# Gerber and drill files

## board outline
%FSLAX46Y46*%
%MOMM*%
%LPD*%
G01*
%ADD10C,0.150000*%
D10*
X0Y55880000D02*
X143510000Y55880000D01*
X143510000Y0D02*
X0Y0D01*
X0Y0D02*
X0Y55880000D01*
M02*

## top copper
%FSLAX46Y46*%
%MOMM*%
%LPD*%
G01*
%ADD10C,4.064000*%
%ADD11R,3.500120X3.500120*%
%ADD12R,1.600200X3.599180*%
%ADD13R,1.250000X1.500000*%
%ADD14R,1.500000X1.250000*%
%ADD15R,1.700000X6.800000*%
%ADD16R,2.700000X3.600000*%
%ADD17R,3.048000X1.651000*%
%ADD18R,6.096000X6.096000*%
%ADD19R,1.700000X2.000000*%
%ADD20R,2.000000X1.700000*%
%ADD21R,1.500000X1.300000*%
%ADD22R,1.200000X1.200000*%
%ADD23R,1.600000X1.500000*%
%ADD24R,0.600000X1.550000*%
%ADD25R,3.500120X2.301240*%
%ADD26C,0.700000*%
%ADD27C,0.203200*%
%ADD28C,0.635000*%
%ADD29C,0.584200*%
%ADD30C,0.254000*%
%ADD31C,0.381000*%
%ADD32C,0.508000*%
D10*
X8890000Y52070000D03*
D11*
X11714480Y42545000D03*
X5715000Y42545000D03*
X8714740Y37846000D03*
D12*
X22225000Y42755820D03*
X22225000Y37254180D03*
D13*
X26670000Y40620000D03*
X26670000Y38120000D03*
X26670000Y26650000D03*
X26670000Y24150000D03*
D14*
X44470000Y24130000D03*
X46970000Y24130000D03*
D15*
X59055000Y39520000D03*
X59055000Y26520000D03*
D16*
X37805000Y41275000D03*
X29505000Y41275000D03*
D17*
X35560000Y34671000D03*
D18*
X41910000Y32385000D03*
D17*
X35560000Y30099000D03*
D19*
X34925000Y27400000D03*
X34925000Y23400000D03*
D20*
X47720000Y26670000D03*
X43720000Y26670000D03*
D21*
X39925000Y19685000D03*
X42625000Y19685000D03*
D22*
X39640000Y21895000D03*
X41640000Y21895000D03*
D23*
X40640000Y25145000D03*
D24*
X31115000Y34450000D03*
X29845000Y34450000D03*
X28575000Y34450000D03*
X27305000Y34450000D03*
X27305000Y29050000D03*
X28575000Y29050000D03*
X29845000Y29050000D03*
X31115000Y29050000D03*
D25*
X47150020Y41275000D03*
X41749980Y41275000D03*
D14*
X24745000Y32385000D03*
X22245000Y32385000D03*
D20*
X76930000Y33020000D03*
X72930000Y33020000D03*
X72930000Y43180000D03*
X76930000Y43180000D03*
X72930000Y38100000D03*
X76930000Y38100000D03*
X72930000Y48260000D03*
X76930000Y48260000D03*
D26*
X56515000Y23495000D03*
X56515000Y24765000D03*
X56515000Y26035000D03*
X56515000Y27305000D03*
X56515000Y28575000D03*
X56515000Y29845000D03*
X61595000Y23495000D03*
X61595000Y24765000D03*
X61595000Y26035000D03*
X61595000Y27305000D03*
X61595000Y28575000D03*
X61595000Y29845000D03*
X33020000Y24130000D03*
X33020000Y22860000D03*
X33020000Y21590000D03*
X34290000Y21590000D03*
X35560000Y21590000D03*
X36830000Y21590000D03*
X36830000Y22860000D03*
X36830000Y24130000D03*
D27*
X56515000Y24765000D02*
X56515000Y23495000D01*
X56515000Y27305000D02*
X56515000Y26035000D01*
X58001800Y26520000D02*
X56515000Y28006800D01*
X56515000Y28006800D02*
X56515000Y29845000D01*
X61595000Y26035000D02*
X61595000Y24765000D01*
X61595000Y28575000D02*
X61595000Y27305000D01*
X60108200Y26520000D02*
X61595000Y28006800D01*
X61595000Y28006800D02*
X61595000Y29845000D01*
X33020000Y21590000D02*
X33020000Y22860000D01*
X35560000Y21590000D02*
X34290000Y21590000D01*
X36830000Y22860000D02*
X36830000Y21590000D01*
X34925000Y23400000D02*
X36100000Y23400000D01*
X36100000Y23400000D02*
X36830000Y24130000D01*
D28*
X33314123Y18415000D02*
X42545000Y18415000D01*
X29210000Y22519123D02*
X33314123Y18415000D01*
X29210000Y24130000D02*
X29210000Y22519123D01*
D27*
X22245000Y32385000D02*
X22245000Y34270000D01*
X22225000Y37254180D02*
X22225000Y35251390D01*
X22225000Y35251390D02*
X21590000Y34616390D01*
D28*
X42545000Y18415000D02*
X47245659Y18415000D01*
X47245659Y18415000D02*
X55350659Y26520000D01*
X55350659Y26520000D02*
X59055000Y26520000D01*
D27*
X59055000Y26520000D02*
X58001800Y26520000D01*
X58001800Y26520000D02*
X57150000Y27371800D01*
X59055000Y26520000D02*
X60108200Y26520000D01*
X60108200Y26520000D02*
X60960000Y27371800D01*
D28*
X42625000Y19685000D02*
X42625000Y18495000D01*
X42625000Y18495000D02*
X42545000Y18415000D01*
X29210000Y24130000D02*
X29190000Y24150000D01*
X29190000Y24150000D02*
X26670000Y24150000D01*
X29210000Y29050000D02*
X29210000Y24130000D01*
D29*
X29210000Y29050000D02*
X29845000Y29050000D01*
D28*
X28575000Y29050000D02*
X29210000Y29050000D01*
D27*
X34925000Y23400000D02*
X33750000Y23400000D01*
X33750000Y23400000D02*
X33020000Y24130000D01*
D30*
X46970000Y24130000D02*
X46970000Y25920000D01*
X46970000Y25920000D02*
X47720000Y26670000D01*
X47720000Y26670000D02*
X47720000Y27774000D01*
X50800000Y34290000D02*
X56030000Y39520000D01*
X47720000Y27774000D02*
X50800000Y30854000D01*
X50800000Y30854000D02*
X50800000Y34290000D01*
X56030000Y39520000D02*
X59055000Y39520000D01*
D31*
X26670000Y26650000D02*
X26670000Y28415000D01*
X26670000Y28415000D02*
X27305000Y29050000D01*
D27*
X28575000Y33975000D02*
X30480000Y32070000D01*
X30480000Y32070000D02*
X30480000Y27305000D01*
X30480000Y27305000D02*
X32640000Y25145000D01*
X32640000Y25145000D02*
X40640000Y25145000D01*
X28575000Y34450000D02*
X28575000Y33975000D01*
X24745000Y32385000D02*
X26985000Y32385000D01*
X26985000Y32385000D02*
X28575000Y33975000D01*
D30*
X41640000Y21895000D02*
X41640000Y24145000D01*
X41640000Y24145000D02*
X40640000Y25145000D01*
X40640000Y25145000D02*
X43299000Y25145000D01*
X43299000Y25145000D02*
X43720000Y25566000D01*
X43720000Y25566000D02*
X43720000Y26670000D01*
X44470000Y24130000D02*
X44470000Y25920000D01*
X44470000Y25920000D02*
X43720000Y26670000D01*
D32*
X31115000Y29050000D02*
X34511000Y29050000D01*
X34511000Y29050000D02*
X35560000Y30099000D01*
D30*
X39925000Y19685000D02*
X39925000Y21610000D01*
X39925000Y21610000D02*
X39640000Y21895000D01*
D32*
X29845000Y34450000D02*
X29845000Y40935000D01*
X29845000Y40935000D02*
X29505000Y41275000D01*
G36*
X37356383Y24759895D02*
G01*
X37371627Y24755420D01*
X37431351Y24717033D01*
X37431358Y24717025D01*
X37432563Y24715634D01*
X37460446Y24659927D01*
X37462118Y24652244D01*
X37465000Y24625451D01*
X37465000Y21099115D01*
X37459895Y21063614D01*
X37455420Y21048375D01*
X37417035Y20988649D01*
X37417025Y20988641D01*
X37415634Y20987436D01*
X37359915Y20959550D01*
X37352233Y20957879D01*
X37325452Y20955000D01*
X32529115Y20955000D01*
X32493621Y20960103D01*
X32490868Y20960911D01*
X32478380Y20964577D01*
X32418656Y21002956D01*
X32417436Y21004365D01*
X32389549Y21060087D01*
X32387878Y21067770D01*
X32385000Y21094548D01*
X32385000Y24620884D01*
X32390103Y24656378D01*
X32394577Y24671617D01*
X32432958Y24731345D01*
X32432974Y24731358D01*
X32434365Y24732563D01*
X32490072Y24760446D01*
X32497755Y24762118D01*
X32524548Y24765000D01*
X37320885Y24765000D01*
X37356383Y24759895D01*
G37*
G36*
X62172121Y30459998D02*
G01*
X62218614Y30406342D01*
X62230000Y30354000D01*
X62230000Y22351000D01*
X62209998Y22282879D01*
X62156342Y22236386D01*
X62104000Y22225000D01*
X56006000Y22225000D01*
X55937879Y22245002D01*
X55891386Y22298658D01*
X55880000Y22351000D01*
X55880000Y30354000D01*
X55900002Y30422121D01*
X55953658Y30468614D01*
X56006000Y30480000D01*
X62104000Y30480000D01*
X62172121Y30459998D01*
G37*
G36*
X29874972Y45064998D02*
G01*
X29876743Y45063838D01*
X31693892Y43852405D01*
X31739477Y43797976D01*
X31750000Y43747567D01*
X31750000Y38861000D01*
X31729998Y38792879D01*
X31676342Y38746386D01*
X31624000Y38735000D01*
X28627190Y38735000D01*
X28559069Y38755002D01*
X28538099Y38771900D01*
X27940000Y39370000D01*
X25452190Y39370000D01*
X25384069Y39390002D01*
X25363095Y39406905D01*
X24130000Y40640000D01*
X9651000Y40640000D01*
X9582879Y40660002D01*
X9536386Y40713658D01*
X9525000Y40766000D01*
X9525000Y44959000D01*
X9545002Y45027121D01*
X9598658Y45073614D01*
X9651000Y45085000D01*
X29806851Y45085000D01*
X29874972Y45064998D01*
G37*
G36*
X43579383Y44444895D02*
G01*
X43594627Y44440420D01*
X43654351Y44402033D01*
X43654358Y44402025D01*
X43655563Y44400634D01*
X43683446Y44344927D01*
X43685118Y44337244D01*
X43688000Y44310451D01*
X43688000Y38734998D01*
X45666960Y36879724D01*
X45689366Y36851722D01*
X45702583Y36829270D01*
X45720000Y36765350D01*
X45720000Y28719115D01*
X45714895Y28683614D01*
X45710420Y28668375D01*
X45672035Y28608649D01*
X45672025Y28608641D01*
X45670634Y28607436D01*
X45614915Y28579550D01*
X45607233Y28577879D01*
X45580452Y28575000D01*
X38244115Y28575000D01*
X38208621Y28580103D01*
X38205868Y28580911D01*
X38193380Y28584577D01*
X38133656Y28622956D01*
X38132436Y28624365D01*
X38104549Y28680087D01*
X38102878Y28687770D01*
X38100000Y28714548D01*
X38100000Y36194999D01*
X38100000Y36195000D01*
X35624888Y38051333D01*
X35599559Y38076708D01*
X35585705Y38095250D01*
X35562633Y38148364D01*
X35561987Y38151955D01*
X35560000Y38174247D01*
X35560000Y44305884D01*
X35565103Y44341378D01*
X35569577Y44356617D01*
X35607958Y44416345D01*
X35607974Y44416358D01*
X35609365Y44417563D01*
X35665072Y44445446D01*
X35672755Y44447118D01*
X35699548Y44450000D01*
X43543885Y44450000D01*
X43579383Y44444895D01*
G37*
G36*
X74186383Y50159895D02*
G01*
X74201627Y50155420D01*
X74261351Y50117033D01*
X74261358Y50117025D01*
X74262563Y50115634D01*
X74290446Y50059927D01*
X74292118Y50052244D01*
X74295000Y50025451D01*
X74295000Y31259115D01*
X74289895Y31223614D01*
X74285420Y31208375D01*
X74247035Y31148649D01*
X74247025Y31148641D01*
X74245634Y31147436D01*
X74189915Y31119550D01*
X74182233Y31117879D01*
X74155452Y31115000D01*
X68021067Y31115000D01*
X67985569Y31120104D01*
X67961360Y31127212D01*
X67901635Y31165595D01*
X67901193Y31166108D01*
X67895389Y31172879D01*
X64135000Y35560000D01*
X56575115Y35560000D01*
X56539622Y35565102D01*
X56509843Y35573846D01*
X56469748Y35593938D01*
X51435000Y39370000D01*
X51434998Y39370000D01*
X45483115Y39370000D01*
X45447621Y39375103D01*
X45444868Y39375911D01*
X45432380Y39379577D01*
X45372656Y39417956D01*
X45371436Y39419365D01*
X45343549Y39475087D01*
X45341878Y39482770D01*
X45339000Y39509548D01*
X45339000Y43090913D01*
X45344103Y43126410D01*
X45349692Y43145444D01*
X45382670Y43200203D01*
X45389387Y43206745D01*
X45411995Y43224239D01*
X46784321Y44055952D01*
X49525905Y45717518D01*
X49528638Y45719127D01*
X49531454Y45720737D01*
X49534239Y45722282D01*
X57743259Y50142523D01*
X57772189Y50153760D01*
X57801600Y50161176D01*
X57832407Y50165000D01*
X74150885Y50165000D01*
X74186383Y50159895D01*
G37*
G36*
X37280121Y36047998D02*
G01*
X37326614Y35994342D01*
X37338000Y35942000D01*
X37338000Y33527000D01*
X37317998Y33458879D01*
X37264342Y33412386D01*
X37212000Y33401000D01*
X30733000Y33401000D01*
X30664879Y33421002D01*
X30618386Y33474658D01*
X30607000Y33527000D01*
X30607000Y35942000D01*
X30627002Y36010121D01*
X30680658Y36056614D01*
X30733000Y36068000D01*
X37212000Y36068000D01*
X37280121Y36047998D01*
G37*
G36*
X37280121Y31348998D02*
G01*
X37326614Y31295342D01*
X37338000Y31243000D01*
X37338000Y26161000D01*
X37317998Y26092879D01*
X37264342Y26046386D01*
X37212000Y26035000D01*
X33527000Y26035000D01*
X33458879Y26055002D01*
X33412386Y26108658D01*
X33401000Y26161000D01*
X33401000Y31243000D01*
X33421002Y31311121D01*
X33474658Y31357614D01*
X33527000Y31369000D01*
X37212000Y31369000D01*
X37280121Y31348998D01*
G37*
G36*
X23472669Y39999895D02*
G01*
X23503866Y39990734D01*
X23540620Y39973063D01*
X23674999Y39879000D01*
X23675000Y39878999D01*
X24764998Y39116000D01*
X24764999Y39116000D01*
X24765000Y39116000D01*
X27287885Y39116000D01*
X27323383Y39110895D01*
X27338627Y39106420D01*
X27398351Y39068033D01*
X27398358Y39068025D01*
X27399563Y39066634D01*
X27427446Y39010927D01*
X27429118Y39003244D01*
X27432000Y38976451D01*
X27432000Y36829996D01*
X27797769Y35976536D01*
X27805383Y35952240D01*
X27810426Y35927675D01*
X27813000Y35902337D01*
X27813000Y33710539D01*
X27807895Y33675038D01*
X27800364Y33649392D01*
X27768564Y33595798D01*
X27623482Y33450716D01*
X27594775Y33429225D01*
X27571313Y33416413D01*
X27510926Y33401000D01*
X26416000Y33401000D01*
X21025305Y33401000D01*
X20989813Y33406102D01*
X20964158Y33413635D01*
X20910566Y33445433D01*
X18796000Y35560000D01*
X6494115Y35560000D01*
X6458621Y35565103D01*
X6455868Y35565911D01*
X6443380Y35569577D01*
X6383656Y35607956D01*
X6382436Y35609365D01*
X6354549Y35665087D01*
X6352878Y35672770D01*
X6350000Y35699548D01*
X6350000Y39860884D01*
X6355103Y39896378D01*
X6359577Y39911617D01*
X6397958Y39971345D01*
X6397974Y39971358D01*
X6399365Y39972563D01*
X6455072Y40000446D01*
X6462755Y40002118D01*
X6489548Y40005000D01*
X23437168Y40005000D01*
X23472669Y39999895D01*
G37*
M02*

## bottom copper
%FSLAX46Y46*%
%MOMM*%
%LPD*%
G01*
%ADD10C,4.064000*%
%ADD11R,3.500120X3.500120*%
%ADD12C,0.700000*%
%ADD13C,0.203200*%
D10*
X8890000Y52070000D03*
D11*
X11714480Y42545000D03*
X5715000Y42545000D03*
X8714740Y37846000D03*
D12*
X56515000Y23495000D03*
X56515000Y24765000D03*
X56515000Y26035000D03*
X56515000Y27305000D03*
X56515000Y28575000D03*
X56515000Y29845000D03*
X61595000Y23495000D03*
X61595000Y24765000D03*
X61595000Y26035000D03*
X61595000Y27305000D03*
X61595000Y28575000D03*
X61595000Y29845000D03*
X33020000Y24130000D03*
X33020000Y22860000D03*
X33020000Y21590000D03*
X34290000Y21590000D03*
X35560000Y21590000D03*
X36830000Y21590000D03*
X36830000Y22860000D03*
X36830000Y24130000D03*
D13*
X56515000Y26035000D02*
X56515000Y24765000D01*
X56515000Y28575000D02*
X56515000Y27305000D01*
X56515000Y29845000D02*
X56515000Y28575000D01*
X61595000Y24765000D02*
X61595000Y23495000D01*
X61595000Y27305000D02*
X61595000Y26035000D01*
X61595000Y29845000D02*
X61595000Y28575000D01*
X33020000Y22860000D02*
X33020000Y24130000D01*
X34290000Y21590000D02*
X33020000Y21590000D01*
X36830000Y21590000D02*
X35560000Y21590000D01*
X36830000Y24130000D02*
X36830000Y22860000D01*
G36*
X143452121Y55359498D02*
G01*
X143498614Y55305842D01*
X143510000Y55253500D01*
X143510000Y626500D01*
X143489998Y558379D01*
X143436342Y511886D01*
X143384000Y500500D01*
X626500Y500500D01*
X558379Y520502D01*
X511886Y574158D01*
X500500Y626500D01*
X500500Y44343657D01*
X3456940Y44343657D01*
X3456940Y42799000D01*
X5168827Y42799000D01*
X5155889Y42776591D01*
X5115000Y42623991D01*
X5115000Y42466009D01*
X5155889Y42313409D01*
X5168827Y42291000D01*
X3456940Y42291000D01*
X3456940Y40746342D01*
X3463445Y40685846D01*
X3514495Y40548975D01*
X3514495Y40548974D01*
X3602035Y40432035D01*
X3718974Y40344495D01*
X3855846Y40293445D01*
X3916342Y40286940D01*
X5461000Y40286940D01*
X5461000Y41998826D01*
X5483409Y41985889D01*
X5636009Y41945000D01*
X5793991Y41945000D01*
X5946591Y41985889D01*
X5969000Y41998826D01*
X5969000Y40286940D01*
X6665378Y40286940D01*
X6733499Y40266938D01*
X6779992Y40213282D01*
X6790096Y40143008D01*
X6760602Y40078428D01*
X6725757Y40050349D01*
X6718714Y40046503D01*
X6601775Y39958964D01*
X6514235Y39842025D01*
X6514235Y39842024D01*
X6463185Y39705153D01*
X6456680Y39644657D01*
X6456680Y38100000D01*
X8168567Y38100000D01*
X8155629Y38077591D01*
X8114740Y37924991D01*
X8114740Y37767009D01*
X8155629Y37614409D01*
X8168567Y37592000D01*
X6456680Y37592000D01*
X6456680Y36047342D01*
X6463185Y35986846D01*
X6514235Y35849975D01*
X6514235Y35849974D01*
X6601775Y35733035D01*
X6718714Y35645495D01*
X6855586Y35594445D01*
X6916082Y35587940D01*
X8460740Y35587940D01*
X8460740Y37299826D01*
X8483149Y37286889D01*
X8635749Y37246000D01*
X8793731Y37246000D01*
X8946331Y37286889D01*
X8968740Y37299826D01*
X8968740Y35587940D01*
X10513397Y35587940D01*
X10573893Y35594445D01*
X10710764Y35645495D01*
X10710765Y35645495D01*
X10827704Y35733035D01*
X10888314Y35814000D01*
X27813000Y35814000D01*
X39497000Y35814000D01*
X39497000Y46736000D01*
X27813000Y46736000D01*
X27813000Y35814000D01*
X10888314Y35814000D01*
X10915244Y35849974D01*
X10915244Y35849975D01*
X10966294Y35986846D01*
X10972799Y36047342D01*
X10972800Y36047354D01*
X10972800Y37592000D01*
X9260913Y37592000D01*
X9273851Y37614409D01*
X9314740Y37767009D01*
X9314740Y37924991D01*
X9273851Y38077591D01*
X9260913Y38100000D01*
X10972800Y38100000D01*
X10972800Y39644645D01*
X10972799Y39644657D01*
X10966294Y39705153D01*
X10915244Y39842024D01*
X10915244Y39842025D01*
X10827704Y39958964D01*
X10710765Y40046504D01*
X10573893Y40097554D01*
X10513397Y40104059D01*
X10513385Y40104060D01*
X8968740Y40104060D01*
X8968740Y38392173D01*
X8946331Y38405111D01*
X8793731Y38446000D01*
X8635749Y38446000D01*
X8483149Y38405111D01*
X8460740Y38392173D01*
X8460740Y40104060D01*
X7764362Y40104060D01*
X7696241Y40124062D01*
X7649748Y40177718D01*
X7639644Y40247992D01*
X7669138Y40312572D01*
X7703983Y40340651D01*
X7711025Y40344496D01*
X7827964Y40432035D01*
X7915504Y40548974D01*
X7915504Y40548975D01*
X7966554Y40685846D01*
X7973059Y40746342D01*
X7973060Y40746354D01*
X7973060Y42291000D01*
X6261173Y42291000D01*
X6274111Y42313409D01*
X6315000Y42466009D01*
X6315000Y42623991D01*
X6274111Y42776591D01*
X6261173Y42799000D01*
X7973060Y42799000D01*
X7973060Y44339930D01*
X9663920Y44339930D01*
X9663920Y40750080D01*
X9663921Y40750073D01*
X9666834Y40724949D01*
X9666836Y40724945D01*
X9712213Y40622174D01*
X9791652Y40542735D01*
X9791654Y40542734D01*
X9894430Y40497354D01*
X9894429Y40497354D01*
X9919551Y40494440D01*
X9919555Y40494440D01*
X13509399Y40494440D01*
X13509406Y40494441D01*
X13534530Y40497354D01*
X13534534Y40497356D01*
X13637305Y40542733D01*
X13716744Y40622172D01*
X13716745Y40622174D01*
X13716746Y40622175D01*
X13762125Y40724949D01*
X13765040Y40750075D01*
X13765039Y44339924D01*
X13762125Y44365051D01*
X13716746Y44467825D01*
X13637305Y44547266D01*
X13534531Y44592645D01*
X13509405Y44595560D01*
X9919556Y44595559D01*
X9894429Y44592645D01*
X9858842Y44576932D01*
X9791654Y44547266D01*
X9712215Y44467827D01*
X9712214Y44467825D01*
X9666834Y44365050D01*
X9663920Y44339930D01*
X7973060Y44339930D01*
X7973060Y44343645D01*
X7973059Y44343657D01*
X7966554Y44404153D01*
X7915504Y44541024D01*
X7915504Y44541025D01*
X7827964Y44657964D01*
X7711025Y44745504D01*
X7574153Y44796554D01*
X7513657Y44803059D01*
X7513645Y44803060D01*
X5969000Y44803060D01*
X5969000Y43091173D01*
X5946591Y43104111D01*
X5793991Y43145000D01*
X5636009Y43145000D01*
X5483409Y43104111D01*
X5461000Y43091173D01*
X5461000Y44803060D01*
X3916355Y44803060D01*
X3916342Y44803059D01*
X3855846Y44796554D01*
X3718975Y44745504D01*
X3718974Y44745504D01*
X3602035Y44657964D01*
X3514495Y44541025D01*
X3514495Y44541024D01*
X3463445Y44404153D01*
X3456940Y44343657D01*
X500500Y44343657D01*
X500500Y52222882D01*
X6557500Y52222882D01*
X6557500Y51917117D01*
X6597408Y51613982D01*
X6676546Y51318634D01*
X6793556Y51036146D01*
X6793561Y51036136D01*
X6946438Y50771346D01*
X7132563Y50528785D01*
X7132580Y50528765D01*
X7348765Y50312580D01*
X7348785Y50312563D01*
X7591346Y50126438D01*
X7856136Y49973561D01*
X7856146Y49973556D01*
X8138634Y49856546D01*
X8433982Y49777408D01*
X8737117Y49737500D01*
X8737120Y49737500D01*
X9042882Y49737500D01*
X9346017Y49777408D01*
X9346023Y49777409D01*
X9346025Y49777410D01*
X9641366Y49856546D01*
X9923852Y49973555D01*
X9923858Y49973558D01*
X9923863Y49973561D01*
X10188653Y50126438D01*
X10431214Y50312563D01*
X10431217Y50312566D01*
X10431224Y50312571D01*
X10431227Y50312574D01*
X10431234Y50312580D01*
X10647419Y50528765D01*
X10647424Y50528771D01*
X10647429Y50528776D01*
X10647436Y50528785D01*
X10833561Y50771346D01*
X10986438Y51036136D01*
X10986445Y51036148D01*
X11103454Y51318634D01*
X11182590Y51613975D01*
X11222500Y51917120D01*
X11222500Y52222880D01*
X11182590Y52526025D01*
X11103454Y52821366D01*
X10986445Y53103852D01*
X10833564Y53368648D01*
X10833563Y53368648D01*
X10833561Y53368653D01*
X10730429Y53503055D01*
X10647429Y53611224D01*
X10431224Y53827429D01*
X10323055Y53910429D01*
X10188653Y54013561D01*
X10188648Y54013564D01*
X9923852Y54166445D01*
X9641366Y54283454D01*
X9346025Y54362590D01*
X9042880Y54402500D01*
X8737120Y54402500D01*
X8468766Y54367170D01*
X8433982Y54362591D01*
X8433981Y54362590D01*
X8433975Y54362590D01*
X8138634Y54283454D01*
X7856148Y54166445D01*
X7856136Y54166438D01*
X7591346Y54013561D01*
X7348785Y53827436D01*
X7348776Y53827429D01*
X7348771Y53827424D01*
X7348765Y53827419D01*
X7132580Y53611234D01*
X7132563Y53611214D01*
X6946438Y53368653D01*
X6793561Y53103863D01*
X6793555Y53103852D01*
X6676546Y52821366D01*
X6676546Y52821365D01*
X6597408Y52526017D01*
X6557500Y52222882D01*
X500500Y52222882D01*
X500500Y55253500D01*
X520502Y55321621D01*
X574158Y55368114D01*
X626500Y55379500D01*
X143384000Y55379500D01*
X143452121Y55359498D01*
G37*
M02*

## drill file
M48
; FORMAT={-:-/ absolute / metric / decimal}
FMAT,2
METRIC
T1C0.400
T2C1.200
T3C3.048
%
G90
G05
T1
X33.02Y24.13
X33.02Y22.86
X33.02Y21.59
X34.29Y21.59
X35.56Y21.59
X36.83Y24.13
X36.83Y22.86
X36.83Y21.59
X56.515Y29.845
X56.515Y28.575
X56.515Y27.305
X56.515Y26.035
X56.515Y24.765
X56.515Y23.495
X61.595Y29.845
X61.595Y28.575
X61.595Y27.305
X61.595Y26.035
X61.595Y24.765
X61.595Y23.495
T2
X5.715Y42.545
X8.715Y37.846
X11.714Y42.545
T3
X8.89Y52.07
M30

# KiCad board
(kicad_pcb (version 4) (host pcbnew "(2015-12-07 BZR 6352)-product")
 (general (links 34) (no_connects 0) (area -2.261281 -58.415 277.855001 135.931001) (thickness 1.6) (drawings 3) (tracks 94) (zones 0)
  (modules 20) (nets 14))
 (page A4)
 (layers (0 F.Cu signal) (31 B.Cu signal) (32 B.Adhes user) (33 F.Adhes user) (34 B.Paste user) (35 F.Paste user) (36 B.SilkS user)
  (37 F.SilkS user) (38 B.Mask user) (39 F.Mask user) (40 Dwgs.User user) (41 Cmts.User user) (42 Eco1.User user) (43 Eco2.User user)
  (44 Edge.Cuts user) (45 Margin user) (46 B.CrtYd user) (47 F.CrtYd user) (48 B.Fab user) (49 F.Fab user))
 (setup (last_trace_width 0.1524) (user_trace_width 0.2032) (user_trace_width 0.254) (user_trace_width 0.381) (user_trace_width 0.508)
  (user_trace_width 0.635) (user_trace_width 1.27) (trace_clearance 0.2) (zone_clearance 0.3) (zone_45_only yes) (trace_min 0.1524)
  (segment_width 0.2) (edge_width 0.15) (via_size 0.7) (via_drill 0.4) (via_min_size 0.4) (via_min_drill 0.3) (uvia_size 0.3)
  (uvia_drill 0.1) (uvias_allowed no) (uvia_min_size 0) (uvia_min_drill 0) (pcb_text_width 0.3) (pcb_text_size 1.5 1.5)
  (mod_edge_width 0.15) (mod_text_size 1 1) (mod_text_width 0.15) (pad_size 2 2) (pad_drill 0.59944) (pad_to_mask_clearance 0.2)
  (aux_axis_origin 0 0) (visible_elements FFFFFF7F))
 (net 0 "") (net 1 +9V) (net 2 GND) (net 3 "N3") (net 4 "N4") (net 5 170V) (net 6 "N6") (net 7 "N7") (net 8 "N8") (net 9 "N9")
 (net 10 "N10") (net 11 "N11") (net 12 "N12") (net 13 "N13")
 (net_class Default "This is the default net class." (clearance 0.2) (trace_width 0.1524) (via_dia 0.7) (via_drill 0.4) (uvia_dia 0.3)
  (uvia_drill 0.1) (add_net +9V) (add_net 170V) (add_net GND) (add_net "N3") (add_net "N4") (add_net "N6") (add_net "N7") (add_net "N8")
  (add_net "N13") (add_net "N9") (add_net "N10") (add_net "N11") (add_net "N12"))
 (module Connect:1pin (layer F.Cu) (at 8.89 -52.07)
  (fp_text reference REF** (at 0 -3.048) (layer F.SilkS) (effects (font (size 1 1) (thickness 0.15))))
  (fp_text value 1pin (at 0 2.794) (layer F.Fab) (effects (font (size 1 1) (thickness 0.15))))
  (pad 1 thru_hole circle (at 0 0) (size 4.064 4.064) (drill 3.048) (layers *.Cu *.Mask F.SilkS)))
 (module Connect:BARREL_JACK (layer F.Cu) (at 5.51434 -42.545)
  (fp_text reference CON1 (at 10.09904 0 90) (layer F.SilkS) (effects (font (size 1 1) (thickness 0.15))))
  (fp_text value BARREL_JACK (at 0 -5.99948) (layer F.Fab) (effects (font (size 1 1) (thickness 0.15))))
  (pad 1 thru_hole rect (at 6.20014 0) (size 3.50012 3.50012) (drill 1.2) (layers *.Cu *.Mask F.SilkS) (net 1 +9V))
  (pad 2 thru_hole rect (at 0.20066 0) (size 3.50012 3.50012) (drill 1.2) (layers *.Cu *.Mask F.SilkS) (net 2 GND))
  (pad 3 thru_hole rect (at 3.2004 4.699) (size 3.50012 3.50012) (drill 1.2) (layers *.Cu *.Mask F.SilkS) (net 2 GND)))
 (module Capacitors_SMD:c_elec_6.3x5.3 (layer F.Cu) (at 22.225 -40.005 90)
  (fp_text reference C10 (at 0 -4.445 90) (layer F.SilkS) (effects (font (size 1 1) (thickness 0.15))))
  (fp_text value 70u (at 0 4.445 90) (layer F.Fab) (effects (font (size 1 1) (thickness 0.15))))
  (pad 1 smd rect (at 2.75082 0 90) (size 3.59918 1.6002) (layers F.Cu F.Paste F.Mask) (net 1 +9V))
  (pad 2 smd rect (at -2.75082 0 90) (size 3.59918 1.6002) (layers F.Cu F.Paste F.Mask) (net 2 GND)))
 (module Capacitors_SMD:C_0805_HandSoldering (layer F.Cu) (at 26.67 -39.37 270)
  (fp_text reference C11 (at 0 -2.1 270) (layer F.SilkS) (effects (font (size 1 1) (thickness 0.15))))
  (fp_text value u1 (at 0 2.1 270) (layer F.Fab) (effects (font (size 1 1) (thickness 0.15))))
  (pad 1 smd rect (at -1.25 0 270) (size 1.5 1.25) (layers F.Cu F.Paste F.Mask) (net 1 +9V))
  (pad 2 smd rect (at 1.25 0 270) (size 1.5 1.25) (layers F.Cu F.Paste F.Mask) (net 2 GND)))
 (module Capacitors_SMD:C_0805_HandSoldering (layer F.Cu) (at 26.67 -25.4 270)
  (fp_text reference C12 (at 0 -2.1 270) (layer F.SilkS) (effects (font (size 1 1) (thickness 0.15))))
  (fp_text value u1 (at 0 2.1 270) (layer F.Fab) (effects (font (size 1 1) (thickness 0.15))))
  (pad 1 smd rect (at -1.25 0 270) (size 1.5 1.25) (layers F.Cu F.Paste F.Mask) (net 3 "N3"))
  (pad 2 smd rect (at 1.25 0 270) (size 1.5 1.25) (layers F.Cu F.Paste F.Mask) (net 2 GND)))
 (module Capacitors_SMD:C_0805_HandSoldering (layer F.Cu) (at 45.72 -24.13)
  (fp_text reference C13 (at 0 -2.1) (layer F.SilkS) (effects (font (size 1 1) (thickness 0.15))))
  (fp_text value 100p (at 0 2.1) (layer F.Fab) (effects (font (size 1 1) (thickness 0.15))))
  (pad 1 smd rect (at -1.25 0) (size 1.5 1.25) (layers F.Cu F.Paste F.Mask) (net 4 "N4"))
  (pad 2 smd rect (at 1.25 0) (size 1.5 1.25) (layers F.Cu F.Paste F.Mask) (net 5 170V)))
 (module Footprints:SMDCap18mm (layer F.Cu) (at 59.055 -33.02 180)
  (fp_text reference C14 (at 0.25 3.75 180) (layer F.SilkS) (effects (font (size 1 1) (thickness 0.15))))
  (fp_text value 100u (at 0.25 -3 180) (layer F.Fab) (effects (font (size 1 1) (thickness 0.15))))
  (pad 1 smd rect (at 0 6.5 180) (size 1.7 6.8) (layers F.Cu F.Paste F.Mask) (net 5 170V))
  (pad 2 smd rect (at 0 -6.5 180) (size 1.7 6.8) (layers F.Cu F.Paste F.Mask) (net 2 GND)))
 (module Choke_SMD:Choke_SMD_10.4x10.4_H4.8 (layer F.Cu) (at 33.655 -41.275 180)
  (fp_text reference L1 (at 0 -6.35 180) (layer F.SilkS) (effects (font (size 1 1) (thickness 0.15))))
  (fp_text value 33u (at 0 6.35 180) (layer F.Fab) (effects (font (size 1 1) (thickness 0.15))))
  (pad 1 smd rect (at -4.15 0 180) (size 2.7 3.6) (layers F.Cu F.Paste F.Mask) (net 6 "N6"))
  (pad 2 smd rect (at 4.15 0 180) (size 2.7 3.6) (layers F.Cu F.Paste F.Mask) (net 1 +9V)))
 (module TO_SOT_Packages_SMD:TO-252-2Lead (layer F.Cu) (at 35.56 -32.385 270)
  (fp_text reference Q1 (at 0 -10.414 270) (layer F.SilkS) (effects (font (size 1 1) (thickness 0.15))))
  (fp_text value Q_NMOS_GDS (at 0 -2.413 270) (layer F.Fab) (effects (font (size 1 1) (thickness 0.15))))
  (pad 1 smd rect (at -2.286 0 270) (size 1.651 3.048) (layers F.Cu F.Paste F.Mask) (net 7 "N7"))
  (pad 2 smd rect (at 0 -6.35 270) (size 6.096 6.096) (layers F.Cu F.Paste F.Mask) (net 6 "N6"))
  (pad 3 smd rect (at 2.286 0 270) (size 1.651 3.048) (layers F.Cu F.Paste F.Mask) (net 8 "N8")))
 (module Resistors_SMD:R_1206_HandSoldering (layer F.Cu) (at 34.925 -25.4 270)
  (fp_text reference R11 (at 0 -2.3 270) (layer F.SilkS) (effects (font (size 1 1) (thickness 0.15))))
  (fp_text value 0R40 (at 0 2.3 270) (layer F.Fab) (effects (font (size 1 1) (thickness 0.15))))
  (pad 1 smd rect (at -2 0 270) (size 2 1.7) (layers F.Cu F.Paste F.Mask) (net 8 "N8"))
  (pad 2 smd rect (at 2 0 270) (size 2 1.7) (layers F.Cu F.Paste F.Mask) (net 2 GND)))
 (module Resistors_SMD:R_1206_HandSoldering (layer F.Cu) (at 45.72 -26.67 180)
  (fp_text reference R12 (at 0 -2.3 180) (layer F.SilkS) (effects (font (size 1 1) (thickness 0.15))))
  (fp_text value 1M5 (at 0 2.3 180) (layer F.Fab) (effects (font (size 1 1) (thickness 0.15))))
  (pad 1 smd rect (at -2 0 180) (size 2 1.7) (layers F.Cu F.Paste F.Mask) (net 5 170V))
  (pad 2 smd rect (at 2 0 180) (size 2 1.7) (layers F.Cu F.Paste F.Mask) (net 4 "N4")))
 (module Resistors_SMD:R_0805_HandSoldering (layer F.Cu) (at 41.275 -19.685)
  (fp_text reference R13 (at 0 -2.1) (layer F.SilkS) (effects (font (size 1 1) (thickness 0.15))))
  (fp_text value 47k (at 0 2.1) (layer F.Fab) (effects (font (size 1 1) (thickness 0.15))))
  (pad 1 smd rect (at -1.35 0) (size 1.5 1.3) (layers F.Cu F.Paste F.Mask) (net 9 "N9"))
  (pad 2 smd rect (at 1.35 0) (size 1.5 1.3) (layers F.Cu F.Paste F.Mask) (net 2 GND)))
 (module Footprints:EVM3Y (layer F.Cu) (at 40.64 -23.495)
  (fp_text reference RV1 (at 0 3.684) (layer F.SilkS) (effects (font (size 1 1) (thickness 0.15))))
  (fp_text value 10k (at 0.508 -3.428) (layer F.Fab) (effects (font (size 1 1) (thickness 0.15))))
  (pad 1 smd rect (at -1 1.6) (size 1.2 1.2) (layers F.Cu F.Paste F.Mask) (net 9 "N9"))
  (pad 3 smd rect (at 1 1.6) (size 1.2 1.2) (layers F.Cu F.Paste F.Mask) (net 4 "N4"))
  (pad 2 smd rect (at 0 -1.65) (size 1.6 1.5) (layers F.Cu F.Paste F.Mask) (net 4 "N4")))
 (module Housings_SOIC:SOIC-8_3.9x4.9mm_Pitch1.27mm (layer F.Cu) (at 29.21 -31.75 270)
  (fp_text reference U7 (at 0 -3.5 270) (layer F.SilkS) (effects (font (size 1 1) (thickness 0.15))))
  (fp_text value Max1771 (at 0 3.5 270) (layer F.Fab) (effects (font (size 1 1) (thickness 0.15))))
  (pad 1 smd rect (at -2.7 -1.905 270) (size 1.55 0.6) (layers F.Cu F.Paste F.Mask) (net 7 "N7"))
  (pad 2 smd rect (at -2.7 -0.635 270) (size 1.55 0.6) (layers F.Cu F.Paste F.Mask) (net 1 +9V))
  (pad 3 smd rect (at -2.7 0.635 270) (size 1.55 0.6) (layers F.Cu F.Paste F.Mask) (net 4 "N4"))
  (pad 4 smd rect (at -2.7 1.905 270) (size 1.55 0.6) (layers F.Cu F.Paste F.Mask) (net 2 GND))
  (pad 5 smd rect (at 2.7 1.905 270) (size 1.55 0.6) (layers F.Cu F.Paste F.Mask) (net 3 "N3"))
  (pad 6 smd rect (at 2.7 0.635 270) (size 1.55 0.6) (layers F.Cu F.Paste F.Mask) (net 2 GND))
  (pad 7 smd rect (at 2.7 -0.635 270) (size 1.55 0.6) (layers F.Cu F.Paste F.Mask) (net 2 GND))
  (pad 8 smd rect (at 2.7 -1.905 270) (size 1.55 0.6) (layers F.Cu F.Paste F.Mask) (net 8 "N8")))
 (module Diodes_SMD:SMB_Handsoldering (layer F.Cu) (at 44.45 -41.275 180)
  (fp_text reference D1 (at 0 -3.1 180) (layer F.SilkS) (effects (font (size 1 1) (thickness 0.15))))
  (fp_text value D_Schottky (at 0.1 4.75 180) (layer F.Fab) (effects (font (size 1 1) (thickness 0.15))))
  (pad 1 smd rect (at -2.70002 0 180) (size 3.50012 2.30124) (layers F.Cu F.Paste F.Mask) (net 5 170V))
  (pad 2 smd rect (at 2.70002 0 180) (size 3.50012 2.30124) (layers F.Cu F.Paste F.Mask) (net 6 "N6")))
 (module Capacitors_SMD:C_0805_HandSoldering (layer F.Cu) (at 23.495 -32.385 180)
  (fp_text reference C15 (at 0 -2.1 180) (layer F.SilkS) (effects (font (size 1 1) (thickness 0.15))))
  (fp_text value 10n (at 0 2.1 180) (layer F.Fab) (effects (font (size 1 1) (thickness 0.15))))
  (pad 1 smd rect (at -1.25 0 180) (size 1.5 1.25) (layers F.Cu F.Paste F.Mask) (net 4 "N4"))
  (pad 2 smd rect (at 1.25 0 180) (size 1.5 1.25) (layers F.Cu F.Paste F.Mask) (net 2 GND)))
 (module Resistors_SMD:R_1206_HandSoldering (layer F.Cu) (at 74.93 -33.02 180)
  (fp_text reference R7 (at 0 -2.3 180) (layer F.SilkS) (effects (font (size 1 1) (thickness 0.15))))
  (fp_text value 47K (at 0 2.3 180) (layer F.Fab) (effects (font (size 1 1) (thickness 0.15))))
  (pad 1 smd rect (at -2 0 180) (size 2 1.7) (layers F.Cu F.Paste F.Mask) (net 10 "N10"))
  (pad 2 smd rect (at 2 0 180) (size 2 1.7) (layers F.Cu F.Paste F.Mask) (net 5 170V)))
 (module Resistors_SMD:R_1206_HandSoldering (layer F.Cu) (at 74.93 -43.18)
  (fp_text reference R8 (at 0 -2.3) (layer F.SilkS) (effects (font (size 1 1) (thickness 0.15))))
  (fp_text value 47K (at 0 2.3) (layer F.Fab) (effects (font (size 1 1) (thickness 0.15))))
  (pad 1 smd rect (at -2 0) (size 2 1.7) (layers F.Cu F.Paste F.Mask) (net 5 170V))
  (pad 2 smd rect (at 2 0) (size 2 1.7) (layers F.Cu F.Paste F.Mask) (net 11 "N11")))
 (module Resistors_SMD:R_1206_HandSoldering (layer F.Cu) (at 74.93 -38.1)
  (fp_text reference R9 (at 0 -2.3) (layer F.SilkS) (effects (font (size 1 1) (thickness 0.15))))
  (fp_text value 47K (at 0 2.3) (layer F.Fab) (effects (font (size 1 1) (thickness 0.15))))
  (pad 1 smd rect (at -2 0) (size 2 1.7) (layers F.Cu F.Paste F.Mask) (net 5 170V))
  (pad 2 smd rect (at 2 0) (size 2 1.7) (layers F.Cu F.Paste F.Mask) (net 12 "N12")))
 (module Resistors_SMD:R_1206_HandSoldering (layer F.Cu) (at 74.93 -48.26)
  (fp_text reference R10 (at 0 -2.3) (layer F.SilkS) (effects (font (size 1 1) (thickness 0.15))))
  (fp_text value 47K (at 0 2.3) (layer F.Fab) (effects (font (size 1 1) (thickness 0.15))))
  (pad 1 smd rect (at -2 0) (size 2 1.7) (layers F.Cu F.Paste F.Mask) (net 5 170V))
  (pad 2 smd rect (at 2 0) (size 2 1.7) (layers F.Cu F.Paste F.Mask) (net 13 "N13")))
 (gr_line (start 0 -55.88) (end 143.51 -55.88) (layer Edge.Cuts) (width 0.15))
 (gr_line (start 143.51 0) (end 0 0) (layer Edge.Cuts) (width 0.15))
 (gr_line (start 0 0) (end 0 -55.88) (layer Edge.Cuts) (width 0.15))
 (segment (start 56.515 -24.765) (end 56.515 -23.495) (width 0.2032) (layer F.Cu) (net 2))
 (via (at 56.515 -23.495) (size 0.7) (drill 0.4) (layers F.Cu B.Cu) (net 2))
 (segment (start 56.515 -26.035) (end 56.515 -24.765) (width 0.2032) (layer B.Cu) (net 2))
 (via (at 56.515 -24.765) (size 0.7) (drill 0.4) (layers F.Cu B.Cu) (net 2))
 (segment (start 56.515 -27.305) (end 56.515 -26.035) (width 0.2032) (layer F.Cu) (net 2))
 (via (at 56.515 -26.035) (size 0.7) (drill 0.4) (layers F.Cu B.Cu) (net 2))
 (segment (start 56.515 -28.575) (end 56.515 -27.305) (width 0.2032) (layer B.Cu) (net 2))
 (via (at 56.515 -27.305) (size 0.7) (drill 0.4) (layers F.Cu B.Cu) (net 2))
 (segment (start 56.515 -29.845) (end 56.515 -28.575) (width 0.2032) (layer B.Cu) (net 2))
 (via (at 56.515 -28.575) (size 0.7) (drill 0.4) (layers F.Cu B.Cu) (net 2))
 (segment (start 58.0018 -26.52) (end 56.515 -28.0068) (width 0.2032) (layer F.Cu) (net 2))
 (segment (start 56.515 -28.0068) (end 56.515 -29.845) (width 0.2032) (layer F.Cu) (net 2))
 (via (at 56.515 -29.845) (size 0.7) (drill 0.4) (layers F.Cu B.Cu) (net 2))
 (segment (start 61.595 -24.765) (end 61.595 -23.495) (width 0.2032) (layer B.Cu) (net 2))
 (via (at 61.595 -23.495) (size 0.7) (drill 0.4) (layers F.Cu B.Cu) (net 2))
 (segment (start 61.595 -26.035) (end 61.595 -24.765) (width 0.2032) (layer F.Cu) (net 2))
 (via (at 61.595 -24.765) (size 0.7) (drill 0.4) (layers F.Cu B.Cu) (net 2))
 (segment (start 61.595 -27.305) (end 61.595 -26.035) (width 0.2032) (layer B.Cu) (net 2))
 (via (at 61.595 -26.035) (size 0.7) (drill 0.4) (layers F.Cu B.Cu) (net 2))
 (segment (start 61.595 -28.575) (end 61.595 -27.305) (width 0.2032) (layer F.Cu) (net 2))
 (via (at 61.595 -27.305) (size 0.7) (drill 0.4) (layers F.Cu B.Cu) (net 2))
 (segment (start 61.595 -29.845) (end 61.595 -28.575) (width 0.2032) (layer B.Cu) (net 2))
 (via (at 61.595 -28.575) (size 0.7) (drill 0.4) (layers F.Cu B.Cu) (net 2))
 (segment (start 60.1082 -26.52) (end 61.595 -28.0068) (width 0.2032) (layer F.Cu) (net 2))
 (segment (start 61.595 -28.0068) (end 61.595 -29.845) (width 0.2032) (layer F.Cu) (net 2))
 (via (at 61.595 -29.845) (size 0.7) (drill 0.4) (layers F.Cu B.Cu) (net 2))
 (segment (start 33.02 -22.86) (end 33.02 -24.13) (width 0.2032) (layer B.Cu) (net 2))
 (via (at 33.02 -24.13) (size 0.7) (drill 0.4) (layers F.Cu B.Cu) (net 2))
 (segment (start 33.02 -21.59) (end 33.02 -22.86) (width 0.2032) (layer F.Cu) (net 2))
 (via (at 33.02 -22.86) (size 0.7) (drill 0.4) (layers F.Cu B.Cu) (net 2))
 (segment (start 34.29 -21.59) (end 33.02 -21.59) (width 0.2032) (layer B.Cu) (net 2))
 (via (at 33.02 -21.59) (size 0.7) (drill 0.4) (layers F.Cu B.Cu) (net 2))
 (segment (start 35.56 -21.59) (end 34.29 -21.59) (width 0.2032) (layer F.Cu) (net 2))
 (via (at 34.29 -21.59) (size 0.7) (drill 0.4) (layers F.Cu B.Cu) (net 2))
 (segment (start 36.83 -21.59) (end 35.56 -21.59) (width 0.2032) (layer B.Cu) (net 2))
 (via (at 35.56 -21.59) (size 0.7) (drill 0.4) (layers F.Cu B.Cu) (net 2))
 (segment (start 36.83 -22.86) (end 36.83 -21.59) (width 0.2032) (layer F.Cu) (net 2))
 (via (at 36.83 -21.59) (size 0.7) (drill 0.4) (layers F.Cu B.Cu) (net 2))
 (segment (start 36.83 -24.13) (end 36.83 -22.86) (width 0.2032) (layer B.Cu) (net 2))
 (via (at 36.83 -22.86) (size 0.7) (drill 0.4) (layers F.Cu B.Cu) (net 2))
 (segment (start 34.925 -23.4) (end 36.1 -23.4) (width 0.2032) (layer F.Cu) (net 2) (status 10))
 (segment (start 36.1 -23.4) (end 36.83 -24.13) (width 0.2032) (layer F.Cu) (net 2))
 (via (at 36.83 -24.13) (size 0.7) (drill 0.4) (layers F.Cu B.Cu) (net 2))
 (segment (start 33.314123 -18.415) (end 42.545 -18.415) (width 0.635) (layer F.Cu) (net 2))
 (segment (start 29.21 -22.519123) (end 33.314123 -18.415) (width 0.635) (layer F.Cu) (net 2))
 (segment (start 29.21 -24.13) (end 29.21 -22.519123) (width 0.635) (layer F.Cu) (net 2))
 (segment (start 22.245 -32.385) (end 22.245 -34.27) (width 0.2032) (layer F.Cu) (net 2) (status 10))
 (segment (start 22.225 -37.25418) (end 22.225 -35.25139) (width 0.2032) (layer F.Cu) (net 2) (status 10))
 (segment (start 22.225 -35.25139) (end 21.59 -34.61639) (width 0.2032) (layer F.Cu) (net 2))
 (segment (start 42.545 -18.415) (end 47.245659 -18.415) (width 0.635) (layer F.Cu) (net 2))
 (segment (start 47.245659 -18.415) (end 55.350659 -26.52) (width 0.635) (layer F.Cu) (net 2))
 (segment (start 55.350659 -26.52) (end 59.055 -26.52) (width 0.635) (layer F.Cu) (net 2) (status 20))
 (segment (start 59.055 -26.52) (end 58.0018 -26.52) (width 0.2032) (layer F.Cu) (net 2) (status 10))
 (segment (start 58.0018 -26.52) (end 57.15 -27.3718) (width 0.2032) (layer F.Cu) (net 2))
 (segment (start 59.055 -26.52) (end 60.1082 -26.52) (width 0.2032) (layer F.Cu) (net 2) (status 10))
 (segment (start 60.1082 -26.52) (end 60.96 -27.3718) (width 0.2032) (layer F.Cu) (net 2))
 (segment (start 42.625 -19.685) (end 42.625 -18.495) (width 0.635) (layer F.Cu) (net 2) (status 10))
 (segment (start 42.625 -18.495) (end 42.545 -18.415) (width 0.635) (layer F.Cu) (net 2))
 (segment (start 29.21 -24.13) (end 29.19 -24.15) (width 0.635) (layer F.Cu) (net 2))
 (segment (start 29.19 -24.15) (end 26.67 -24.15) (width 0.635) (layer F.Cu) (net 2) (status 20))
 (segment (start 29.21 -29.05) (end 29.21 -24.13) (width 0.635) (layer F.Cu) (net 2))
 (segment (start 29.21 -29.05) (end 29.845 -29.05) (width 0.5842) (layer F.Cu) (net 2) (status 20))
 (segment (start 28.575 -29.05) (end 29.21 -29.05) (width 0.635) (layer F.Cu) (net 2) (status 10))
 (segment (start 34.925 -23.4) (end 33.75 -23.4) (width 0.2032) (layer F.Cu) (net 2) (status 10))
 (segment (start 33.75 -23.4) (end 33.02 -24.13) (width 0.2032) (layer F.Cu) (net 2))
 (segment (start 46.97 -24.13) (end 46.97 -25.92) (width 0.254) (layer F.Cu) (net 5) (status 30))
 (segment (start 46.97 -25.92) (end 47.72 -26.67) (width 0.254) (layer F.Cu) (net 5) (status 30))
 (segment (start 47.72 -26.67) (end 47.72 -27.774) (width 0.254) (layer F.Cu) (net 5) (status 10))
 (segment (start 50.8 -34.29) (end 56.03 -39.52) (width 0.254) (layer F.Cu) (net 5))
 (segment (start 47.72 -27.774) (end 50.8 -30.854) (width 0.254) (layer F.Cu) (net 5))
 (segment (start 50.8 -30.854) (end 50.8 -34.29) (width 0.254) (layer F.Cu) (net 5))
 (segment (start 56.03 -39.52) (end 59.055 -39.52) (width 0.254) (layer F.Cu) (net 5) (status 20))
 (segment (start 26.67 -26.65) (end 26.67 -28.415) (width 0.381) (layer F.Cu) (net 3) (status 10))
 (segment (start 26.67 -28.415) (end 27.305 -29.05) (width 0.381) (layer F.Cu) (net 3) (status 20))
 (segment (start 28.575 -33.975) (end 30.48 -32.07) (width 0.2032) (layer F.Cu) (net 4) (status 10))
 (segment (start 30.48 -32.07) (end 30.48 -27.305) (width 0.2032) (layer F.Cu) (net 4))
 (segment (start 30.48 -27.305) (end 32.64 -25.145) (width 0.2032) (layer F.Cu) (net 4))
 (segment (start 32.64 -25.145) (end 40.64 -25.145) (width 0.2032) (layer F.Cu) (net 4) (status 20))
 (segment (start 28.575 -34.45) (end 28.575 -33.975) (width 0.2032) (layer F.Cu) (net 4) (status 30))
 (segment (start 24.745 -32.385) (end 26.985 -32.385) (width 0.2032) (layer F.Cu) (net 4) (status 10))
 (segment (start 26.985 -32.385) (end 28.575 -33.975) (width 0.2032) (layer F.Cu) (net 4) (status 20))
 (segment (start 41.64 -21.895) (end 41.64 -24.145) (width 0.254) (layer F.Cu) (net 4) (status 10))
 (segment (start 41.64 -24.145) (end 40.64 -25.145) (width 0.254) (layer F.Cu) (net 4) (status 20))
 (segment (start 40.64 -25.145) (end 43.299 -25.145) (width 0.254) (layer F.Cu) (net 4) (status 10))
 (segment (start 43.299 -25.145) (end 43.72 -25.566) (width 0.254) (layer F.Cu) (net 4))
 (segment (start 43.72 -25.566) (end 43.72 -26.67) (width 0.254) (layer F.Cu) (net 4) (status 20))
 (segment (start 44.47 -24.13) (end 44.47 -25.92) (width 0.254) (layer F.Cu) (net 4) (status 30))
 (segment (start 44.47 -25.92) (end 43.72 -26.67) (width 0.254) (layer F.Cu) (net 4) (status 30))
 (segment (start 31.115 -29.05) (end 34.511 -29.05) (width 0.508) (layer F.Cu) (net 8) (status 10))
 (segment (start 34.511 -29.05) (end 35.56 -30.099) (width 0.508) (layer F.Cu) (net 8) (status 20))
 (segment (start 39.925 -19.685) (end 39.925 -21.61) (width 0.254) (layer F.Cu) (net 9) (status 30))
 (segment (start 39.925 -21.61) (end 39.64 -21.895) (width 0.254) (layer F.Cu) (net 9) (status 30))
 (segment (start 29.845 -34.45) (end 29.845 -40.935) (width 0.508) (layer F.Cu) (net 1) (status 30))
 (segment (start 29.845 -40.935) (end 29.505 -41.275) (width 0.508) (layer F.Cu) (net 1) (status 30))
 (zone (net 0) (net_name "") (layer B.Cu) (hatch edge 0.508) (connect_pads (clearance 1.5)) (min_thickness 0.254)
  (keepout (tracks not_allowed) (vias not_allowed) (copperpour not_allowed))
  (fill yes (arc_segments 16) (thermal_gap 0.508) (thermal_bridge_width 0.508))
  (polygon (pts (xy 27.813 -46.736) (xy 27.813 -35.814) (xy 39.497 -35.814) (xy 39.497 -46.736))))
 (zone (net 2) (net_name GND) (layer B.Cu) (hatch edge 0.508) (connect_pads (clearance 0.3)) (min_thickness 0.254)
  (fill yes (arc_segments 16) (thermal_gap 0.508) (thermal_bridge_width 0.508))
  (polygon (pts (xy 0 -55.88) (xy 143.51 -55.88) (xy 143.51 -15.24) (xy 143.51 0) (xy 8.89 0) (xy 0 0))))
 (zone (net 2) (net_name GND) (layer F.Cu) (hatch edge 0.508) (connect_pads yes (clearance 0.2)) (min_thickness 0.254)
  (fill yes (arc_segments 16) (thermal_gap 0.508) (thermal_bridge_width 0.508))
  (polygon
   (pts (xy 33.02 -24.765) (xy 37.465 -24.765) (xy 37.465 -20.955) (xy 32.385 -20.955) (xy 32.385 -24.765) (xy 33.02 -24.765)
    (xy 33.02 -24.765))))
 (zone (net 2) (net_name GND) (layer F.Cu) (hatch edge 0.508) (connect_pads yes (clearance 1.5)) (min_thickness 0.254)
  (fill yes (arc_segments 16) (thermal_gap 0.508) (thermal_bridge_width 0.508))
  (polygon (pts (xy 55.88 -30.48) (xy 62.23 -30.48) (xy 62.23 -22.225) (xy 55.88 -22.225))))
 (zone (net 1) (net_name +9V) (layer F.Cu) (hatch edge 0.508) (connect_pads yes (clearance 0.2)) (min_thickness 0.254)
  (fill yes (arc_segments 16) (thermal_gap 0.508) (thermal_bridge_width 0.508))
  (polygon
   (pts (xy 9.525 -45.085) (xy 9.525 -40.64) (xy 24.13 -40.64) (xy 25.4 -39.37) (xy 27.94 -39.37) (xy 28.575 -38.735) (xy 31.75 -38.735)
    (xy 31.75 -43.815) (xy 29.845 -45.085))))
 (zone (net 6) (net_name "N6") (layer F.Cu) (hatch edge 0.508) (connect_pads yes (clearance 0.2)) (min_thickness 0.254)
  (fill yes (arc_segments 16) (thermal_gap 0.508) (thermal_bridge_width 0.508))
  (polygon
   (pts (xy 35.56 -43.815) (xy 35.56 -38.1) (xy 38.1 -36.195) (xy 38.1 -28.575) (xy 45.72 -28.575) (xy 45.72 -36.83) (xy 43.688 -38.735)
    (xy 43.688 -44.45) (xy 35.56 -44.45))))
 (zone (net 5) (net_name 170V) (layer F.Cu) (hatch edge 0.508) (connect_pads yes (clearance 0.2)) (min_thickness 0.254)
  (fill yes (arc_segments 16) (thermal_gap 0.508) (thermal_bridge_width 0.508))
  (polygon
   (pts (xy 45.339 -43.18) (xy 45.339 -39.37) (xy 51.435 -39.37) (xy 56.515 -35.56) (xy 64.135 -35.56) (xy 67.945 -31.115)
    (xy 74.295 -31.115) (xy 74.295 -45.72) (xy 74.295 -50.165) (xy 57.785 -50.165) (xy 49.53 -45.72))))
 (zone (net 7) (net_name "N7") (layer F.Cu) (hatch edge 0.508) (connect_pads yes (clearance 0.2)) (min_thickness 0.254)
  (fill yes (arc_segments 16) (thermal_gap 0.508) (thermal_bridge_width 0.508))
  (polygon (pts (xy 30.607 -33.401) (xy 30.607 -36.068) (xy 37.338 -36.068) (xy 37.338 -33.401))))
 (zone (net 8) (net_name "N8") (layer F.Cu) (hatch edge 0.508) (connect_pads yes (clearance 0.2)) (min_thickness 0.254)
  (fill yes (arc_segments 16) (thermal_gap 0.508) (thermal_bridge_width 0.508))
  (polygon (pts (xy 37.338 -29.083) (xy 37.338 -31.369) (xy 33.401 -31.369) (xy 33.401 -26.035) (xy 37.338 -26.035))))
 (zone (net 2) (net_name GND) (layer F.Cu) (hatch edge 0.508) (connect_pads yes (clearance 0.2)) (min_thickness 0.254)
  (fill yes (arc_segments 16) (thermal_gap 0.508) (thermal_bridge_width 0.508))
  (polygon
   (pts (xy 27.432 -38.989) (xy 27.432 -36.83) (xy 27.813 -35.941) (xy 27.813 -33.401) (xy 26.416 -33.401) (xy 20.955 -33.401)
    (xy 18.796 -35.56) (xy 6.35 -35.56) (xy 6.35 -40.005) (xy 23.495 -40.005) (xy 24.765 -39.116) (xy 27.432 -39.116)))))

